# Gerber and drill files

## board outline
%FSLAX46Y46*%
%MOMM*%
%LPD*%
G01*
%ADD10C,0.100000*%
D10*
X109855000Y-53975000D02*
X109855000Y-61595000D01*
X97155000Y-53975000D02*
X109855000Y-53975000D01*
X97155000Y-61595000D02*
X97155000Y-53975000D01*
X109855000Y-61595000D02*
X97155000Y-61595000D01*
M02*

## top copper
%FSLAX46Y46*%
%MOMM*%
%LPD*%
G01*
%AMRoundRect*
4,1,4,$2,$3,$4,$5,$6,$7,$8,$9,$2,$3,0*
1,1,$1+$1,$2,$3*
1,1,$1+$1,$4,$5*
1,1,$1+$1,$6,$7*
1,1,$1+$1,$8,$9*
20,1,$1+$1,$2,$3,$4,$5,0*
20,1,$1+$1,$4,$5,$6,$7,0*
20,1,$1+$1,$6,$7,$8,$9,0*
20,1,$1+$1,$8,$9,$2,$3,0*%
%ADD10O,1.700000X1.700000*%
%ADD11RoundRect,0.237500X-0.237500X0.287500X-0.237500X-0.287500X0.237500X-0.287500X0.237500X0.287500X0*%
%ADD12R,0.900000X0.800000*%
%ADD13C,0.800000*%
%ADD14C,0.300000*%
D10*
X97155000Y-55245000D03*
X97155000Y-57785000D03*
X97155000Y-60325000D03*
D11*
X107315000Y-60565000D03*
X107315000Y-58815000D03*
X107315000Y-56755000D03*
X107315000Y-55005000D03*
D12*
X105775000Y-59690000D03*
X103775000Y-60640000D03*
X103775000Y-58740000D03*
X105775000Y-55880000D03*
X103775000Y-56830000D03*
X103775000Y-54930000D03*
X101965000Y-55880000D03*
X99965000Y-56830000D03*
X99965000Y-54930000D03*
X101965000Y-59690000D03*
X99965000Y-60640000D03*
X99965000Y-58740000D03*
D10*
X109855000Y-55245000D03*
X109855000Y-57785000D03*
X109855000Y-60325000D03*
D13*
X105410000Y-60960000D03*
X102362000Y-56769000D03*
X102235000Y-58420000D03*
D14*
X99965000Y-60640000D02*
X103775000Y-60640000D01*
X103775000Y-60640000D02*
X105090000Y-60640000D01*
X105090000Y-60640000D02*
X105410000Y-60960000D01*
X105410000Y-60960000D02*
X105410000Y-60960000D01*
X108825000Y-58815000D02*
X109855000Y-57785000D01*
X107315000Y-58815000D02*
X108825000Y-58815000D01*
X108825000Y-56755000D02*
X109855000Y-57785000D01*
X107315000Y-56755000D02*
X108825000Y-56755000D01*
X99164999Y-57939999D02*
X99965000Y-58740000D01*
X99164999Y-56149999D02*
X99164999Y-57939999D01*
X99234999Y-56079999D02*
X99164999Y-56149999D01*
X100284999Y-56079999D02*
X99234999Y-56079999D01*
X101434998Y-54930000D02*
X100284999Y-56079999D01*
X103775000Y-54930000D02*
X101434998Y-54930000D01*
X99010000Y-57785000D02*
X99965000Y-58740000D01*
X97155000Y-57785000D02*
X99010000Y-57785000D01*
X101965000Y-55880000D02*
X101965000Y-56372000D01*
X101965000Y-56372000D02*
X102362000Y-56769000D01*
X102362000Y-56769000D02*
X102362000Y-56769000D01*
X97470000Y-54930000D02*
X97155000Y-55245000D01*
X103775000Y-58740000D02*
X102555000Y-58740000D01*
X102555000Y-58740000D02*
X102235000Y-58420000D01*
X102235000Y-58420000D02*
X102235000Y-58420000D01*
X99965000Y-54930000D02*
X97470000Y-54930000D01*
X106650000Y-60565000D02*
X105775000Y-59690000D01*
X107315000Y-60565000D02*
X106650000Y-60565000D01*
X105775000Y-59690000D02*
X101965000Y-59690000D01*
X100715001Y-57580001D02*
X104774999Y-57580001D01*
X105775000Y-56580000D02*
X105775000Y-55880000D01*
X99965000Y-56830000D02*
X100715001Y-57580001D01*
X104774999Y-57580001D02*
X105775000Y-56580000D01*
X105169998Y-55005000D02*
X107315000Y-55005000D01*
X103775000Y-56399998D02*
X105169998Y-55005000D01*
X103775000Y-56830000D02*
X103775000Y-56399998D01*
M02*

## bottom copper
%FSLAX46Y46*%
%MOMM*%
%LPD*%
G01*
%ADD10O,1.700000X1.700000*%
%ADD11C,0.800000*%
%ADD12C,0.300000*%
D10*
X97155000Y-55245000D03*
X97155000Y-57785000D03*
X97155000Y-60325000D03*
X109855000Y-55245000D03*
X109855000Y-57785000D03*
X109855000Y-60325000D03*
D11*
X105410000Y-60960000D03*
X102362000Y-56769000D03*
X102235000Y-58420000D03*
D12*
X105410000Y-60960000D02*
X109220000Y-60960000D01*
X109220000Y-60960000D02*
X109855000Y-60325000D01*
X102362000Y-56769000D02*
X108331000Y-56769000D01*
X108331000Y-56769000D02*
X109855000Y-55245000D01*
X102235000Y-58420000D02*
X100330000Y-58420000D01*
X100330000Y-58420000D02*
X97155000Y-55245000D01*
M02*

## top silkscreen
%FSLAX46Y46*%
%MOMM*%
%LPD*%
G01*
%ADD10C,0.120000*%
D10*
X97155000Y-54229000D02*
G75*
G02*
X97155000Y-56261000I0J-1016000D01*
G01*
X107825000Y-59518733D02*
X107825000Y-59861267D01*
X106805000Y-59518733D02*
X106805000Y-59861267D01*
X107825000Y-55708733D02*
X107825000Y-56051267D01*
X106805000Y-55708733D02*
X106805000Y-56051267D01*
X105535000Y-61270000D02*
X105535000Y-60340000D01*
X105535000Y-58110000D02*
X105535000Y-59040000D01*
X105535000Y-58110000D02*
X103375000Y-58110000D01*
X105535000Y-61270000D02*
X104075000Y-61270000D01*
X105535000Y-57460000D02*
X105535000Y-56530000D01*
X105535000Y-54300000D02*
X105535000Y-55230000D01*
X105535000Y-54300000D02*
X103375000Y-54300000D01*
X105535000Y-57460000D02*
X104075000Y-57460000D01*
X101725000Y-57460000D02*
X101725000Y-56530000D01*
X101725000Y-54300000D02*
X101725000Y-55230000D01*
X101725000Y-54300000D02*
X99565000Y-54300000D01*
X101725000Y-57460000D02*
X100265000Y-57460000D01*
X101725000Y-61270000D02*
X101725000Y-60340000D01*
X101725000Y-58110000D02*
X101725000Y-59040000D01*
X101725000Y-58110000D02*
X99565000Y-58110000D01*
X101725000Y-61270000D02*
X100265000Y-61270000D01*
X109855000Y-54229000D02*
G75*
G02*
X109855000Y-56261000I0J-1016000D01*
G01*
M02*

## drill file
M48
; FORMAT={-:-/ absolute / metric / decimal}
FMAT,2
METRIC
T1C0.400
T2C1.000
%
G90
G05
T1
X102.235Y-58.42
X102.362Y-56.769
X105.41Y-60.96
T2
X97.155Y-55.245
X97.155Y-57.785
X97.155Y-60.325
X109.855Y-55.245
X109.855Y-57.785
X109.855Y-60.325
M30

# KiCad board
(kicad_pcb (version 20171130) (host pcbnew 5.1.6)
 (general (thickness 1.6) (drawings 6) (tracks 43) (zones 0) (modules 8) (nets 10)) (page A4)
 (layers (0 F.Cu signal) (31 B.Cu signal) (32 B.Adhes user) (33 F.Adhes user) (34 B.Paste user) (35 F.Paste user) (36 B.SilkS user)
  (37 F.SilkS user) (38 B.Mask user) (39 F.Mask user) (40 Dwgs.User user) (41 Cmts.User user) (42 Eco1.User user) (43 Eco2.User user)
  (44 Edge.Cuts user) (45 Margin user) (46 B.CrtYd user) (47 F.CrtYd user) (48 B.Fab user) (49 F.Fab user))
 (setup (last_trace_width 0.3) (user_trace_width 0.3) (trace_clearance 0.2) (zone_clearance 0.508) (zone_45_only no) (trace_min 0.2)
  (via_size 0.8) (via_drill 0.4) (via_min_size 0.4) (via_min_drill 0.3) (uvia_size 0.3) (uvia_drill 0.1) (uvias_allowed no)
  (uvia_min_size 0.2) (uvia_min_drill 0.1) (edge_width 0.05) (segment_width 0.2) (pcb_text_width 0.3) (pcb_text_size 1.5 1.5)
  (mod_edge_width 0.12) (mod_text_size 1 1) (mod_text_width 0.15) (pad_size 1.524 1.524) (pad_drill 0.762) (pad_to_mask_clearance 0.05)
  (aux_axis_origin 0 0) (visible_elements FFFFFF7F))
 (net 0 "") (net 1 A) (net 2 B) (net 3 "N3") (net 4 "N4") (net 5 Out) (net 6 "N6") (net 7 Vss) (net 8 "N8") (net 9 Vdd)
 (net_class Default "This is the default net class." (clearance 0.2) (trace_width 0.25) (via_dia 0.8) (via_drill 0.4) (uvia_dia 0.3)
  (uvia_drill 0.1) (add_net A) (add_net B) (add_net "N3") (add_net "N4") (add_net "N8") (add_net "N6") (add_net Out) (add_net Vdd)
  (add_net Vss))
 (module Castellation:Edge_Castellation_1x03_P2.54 (layer F.Cu) (at 97.155 55.245)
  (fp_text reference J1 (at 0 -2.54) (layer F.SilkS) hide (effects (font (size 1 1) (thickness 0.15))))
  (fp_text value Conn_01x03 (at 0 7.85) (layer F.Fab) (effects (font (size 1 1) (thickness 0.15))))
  (fp_arc (start 0 0) (end 0 1.016) (angle -180) (layer F.SilkS) (width 0.12))
  (pad 1 thru_hole oval (at 0 0) (size 1.7 1.7) (drill 1) (layers *.Cu *.Mask) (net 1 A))
  (pad 2 thru_hole oval (at 0 2.54) (size 1.7 1.7) (drill 1) (layers *.Cu *.Mask) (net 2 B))
  (pad 3 thru_hole oval (at 0 5.08) (size 1.7 1.7) (drill 1) (layers *.Cu *.Mask) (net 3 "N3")))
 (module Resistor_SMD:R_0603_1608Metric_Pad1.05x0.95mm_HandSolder (layer F.Cu) (at 107.315 59.69 270)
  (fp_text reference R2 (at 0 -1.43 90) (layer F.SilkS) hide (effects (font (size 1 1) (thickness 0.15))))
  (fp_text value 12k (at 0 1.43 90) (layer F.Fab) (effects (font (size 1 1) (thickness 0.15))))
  (fp_line (start -0.171267 -0.51) (end 0.171267 -0.51) (layer F.SilkS) (width 0.12))
  (fp_line (start -0.171267 0.51) (end 0.171267 0.51) (layer F.SilkS) (width 0.12))
  (pad 2 smd roundrect (at 0.875 0 270) (size 1.05 0.95) (layers F.Cu F.Paste F.Mask) (roundrect_rratio 0.25) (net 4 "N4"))
  (pad 1 smd roundrect (at -0.875 0 270) (size 1.05 0.95) (layers F.Cu F.Paste F.Mask) (roundrect_rratio 0.25) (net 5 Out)))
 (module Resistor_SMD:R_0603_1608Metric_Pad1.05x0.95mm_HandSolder (layer F.Cu) (at 107.315 55.88 270)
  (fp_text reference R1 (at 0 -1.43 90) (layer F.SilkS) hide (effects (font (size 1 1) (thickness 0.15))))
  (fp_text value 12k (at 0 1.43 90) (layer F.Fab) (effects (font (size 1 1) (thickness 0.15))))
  (fp_line (start -0.171267 -0.51) (end 0.171267 -0.51) (layer F.SilkS) (width 0.12))
  (fp_line (start -0.171267 0.51) (end 0.171267 0.51) (layer F.SilkS) (width 0.12))
  (pad 2 smd roundrect (at 0.875 0 270) (size 1.05 0.95) (layers F.Cu F.Paste F.Mask) (roundrect_rratio 0.25) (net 5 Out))
  (pad 1 smd roundrect (at -0.875 0 270) (size 1.05 0.95) (layers F.Cu F.Paste F.Mask) (roundrect_rratio 0.25) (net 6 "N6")))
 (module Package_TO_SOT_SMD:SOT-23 (layer F.Cu) (at 104.775 59.69)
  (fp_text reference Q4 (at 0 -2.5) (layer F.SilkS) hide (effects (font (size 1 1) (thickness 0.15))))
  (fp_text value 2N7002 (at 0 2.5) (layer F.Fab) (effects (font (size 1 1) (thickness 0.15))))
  (fp_line (start 0.76 1.58) (end 0.76 0.65) (layer F.SilkS) (width 0.12))
  (fp_line (start 0.76 -1.58) (end 0.76 -0.65) (layer F.SilkS) (width 0.12))
  (fp_line (start 0.76 -1.58) (end -1.4 -1.58) (layer F.SilkS) (width 0.12))
  (fp_line (start 0.76 1.58) (end -0.7 1.58) (layer F.SilkS) (width 0.12))
  (pad 3 smd rect (at 1 0) (size 0.9 0.8) (layers F.Cu F.Paste F.Mask) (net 4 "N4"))
  (pad 2 smd rect (at -1 0.95) (size 0.9 0.8) (layers F.Cu F.Paste F.Mask) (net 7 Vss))
  (pad 1 smd rect (at -1 -0.95) (size 0.9 0.8) (layers F.Cu F.Paste F.Mask) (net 1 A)))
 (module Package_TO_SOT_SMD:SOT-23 (layer F.Cu) (at 104.775 55.88)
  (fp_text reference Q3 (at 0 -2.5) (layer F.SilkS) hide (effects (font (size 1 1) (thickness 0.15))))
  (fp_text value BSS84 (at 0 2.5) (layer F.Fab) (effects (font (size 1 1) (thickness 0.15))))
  (fp_line (start 0.76 1.58) (end 0.76 0.65) (layer F.SilkS) (width 0.12))
  (fp_line (start 0.76 -1.58) (end 0.76 -0.65) (layer F.SilkS) (width 0.12))
  (fp_line (start 0.76 -1.58) (end -1.4 -1.58) (layer F.SilkS) (width 0.12))
  (fp_line (start 0.76 1.58) (end -0.7 1.58) (layer F.SilkS) (width 0.12))
  (pad 3 smd rect (at 1 0) (size 0.9 0.8) (layers F.Cu F.Paste F.Mask) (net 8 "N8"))
  (pad 2 smd rect (at -1 0.95) (size 0.9 0.8) (layers F.Cu F.Paste F.Mask) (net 6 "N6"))
  (pad 1 smd rect (at -1 -0.95) (size 0.9 0.8) (layers F.Cu F.Paste F.Mask) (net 2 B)))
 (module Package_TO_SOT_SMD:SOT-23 (layer F.Cu) (at 100.965 55.88)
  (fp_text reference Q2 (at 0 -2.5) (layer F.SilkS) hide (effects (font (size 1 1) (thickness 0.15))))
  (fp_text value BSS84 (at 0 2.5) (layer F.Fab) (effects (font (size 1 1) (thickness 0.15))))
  (fp_line (start 0.76 1.58) (end 0.76 0.65) (layer F.SilkS) (width 0.12))
  (fp_line (start 0.76 -1.58) (end 0.76 -0.65) (layer F.SilkS) (width 0.12))
  (fp_line (start 0.76 -1.58) (end -1.4 -1.58) (layer F.SilkS) (width 0.12))
  (fp_line (start 0.76 1.58) (end -0.7 1.58) (layer F.SilkS) (width 0.12))
  (pad 3 smd rect (at 1 0) (size 0.9 0.8) (layers F.Cu F.Paste F.Mask) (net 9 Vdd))
  (pad 2 smd rect (at -1 0.95) (size 0.9 0.8) (layers F.Cu F.Paste F.Mask) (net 8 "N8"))
  (pad 1 smd rect (at -1 -0.95) (size 0.9 0.8) (layers F.Cu F.Paste F.Mask) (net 1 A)))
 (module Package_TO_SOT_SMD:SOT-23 (layer F.Cu) (at 100.965 59.69)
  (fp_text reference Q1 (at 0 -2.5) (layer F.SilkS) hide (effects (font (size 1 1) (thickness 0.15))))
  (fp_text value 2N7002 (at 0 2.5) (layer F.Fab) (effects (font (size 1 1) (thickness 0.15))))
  (fp_line (start 0.76 1.58) (end 0.76 0.65) (layer F.SilkS) (width 0.12))
  (fp_line (start 0.76 -1.58) (end 0.76 -0.65) (layer F.SilkS) (width 0.12))
  (fp_line (start 0.76 -1.58) (end -1.4 -1.58) (layer F.SilkS) (width 0.12))
  (fp_line (start 0.76 1.58) (end -0.7 1.58) (layer F.SilkS) (width 0.12))
  (pad 3 smd rect (at 1 0) (size 0.9 0.8) (layers F.Cu F.Paste F.Mask) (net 4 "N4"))
  (pad 2 smd rect (at -1 0.95) (size 0.9 0.8) (layers F.Cu F.Paste F.Mask) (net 7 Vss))
  (pad 1 smd rect (at -1 -0.95) (size 0.9 0.8) (layers F.Cu F.Paste F.Mask) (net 2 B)))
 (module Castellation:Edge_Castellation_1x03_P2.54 (layer F.Cu) (at 109.855 55.245)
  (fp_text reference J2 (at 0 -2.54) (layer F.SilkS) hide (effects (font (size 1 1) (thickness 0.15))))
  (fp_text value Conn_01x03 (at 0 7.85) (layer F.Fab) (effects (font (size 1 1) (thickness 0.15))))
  (fp_arc (start 0 0) (end 0 1.016) (angle -180) (layer F.SilkS) (width 0.12))
  (pad 1 thru_hole oval (at 0 0) (size 1.7 1.7) (drill 1) (layers *.Cu *.Mask) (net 9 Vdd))
  (pad 2 thru_hole oval (at 0 2.54) (size 1.7 1.7) (drill 1) (layers *.Cu *.Mask) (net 5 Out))
  (pad 3 thru_hole oval (at 0 5.08) (size 1.7 1.7) (drill 1) (layers *.Cu *.Mask) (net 7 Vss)))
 (gr_line (start 109.855 53.975) (end 109.855 61.595) (layer Edge.Cuts) (width 0.1))
 (gr_line (start 97.155 53.975) (end 109.855 53.975) (layer Edge.Cuts) (width 0.1))
 (gr_line (start 97.155 61.595) (end 97.155 53.975) (layer Edge.Cuts) (width 0.1))
 (gr_line (start 109.855 61.595) (end 97.155 61.595) (layer Edge.Cuts) (width 0.1))
 (segment (start 99.965 60.64) (end 103.775 60.64) (width 0.3) (layer F.Cu) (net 7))
 (segment (start 103.775 60.64) (end 105.09 60.64) (width 0.3) (layer F.Cu) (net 7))
 (segment (start 105.09 60.64) (end 105.41 60.96) (width 0.3) (layer F.Cu) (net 7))
 (segment (start 105.41 60.96) (end 105.41 60.96) (width 0.3) (layer F.Cu) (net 7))
 (via (at 105.41 60.96) (size 0.8) (drill 0.4) (layers F.Cu B.Cu) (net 7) (status 1000000))
 (segment (start 105.41 60.96) (end 109.22 60.96) (width 0.3) (layer B.Cu) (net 7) (status 1000000))
 (segment (start 109.22 60.96) (end 109.855 60.325) (width 0.3) (layer B.Cu) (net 7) (status 1000000))
 (segment (start 108.825 58.815) (end 109.855 57.785) (width 0.3) (layer F.Cu) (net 5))
 (segment (start 107.315 58.815) (end 108.825 58.815) (width 0.3) (layer F.Cu) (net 5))
 (segment (start 108.825 56.755) (end 109.855 57.785) (width 0.3) (layer F.Cu) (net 5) (status 1000000))
 (segment (start 107.315 56.755) (end 108.825 56.755) (width 0.3) (layer F.Cu) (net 5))
 (segment (start 99.164999 57.939999) (end 99.965 58.74) (width 0.3) (layer F.Cu) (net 2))
 (segment (start 99.164999 56.149999) (end 99.164999 57.939999) (width 0.3) (layer F.Cu) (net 2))
 (segment (start 99.234999 56.079999) (end 99.164999 56.149999) (width 0.3) (layer F.Cu) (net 2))
 (segment (start 100.284999 56.079999) (end 99.234999 56.079999) (width 0.3) (layer F.Cu) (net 2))
 (segment (start 101.434998 54.93) (end 100.284999 56.079999) (width 0.3) (layer F.Cu) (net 2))
 (segment (start 103.775 54.93) (end 101.434998 54.93) (width 0.3) (layer F.Cu) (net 2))
 (segment (start 99.01 57.785) (end 99.965 58.74) (width 0.3) (layer F.Cu) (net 2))
 (segment (start 97.155 57.785) (end 99.01 57.785) (width 0.3) (layer F.Cu) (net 2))
 (segment (start 101.965 55.88) (end 101.965 56.372) (width 0.3) (layer F.Cu) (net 9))
 (segment (start 101.965 56.372) (end 102.362 56.769) (width 0.3) (layer F.Cu) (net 9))
 (segment (start 102.362 56.769) (end 102.362 56.769) (width 0.3) (layer F.Cu) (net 9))
 (via (at 102.362 56.769) (size 0.8) (drill 0.4) (layers F.Cu B.Cu) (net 9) (status 1000000))
 (segment (start 102.362 56.769) (end 108.331 56.769) (width 0.3) (layer B.Cu) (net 9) (status 1000000))
 (segment (start 108.331 56.769) (end 109.855 55.245) (width 0.3) (layer B.Cu) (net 9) (status 1000000))
 (segment (start 97.47 54.93) (end 97.155 55.245) (width 0.3) (layer F.Cu) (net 1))
 (segment (start 103.775 58.74) (end 102.555 58.74) (width 0.3) (layer F.Cu) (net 1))
 (segment (start 102.555 58.74) (end 102.235 58.42) (width 0.3) (layer F.Cu) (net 1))
 (segment (start 102.235 58.42) (end 102.235 58.42) (width 0.3) (layer F.Cu) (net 1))
 (segment (start 99.965 54.93) (end 97.47 54.93) (width 0.3) (layer F.Cu) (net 1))
 (segment (start 102.235 58.42) (end 100.33 58.42) (width 0.3) (layer B.Cu) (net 1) (status 1000000))
 (via (at 102.235 58.42) (size 0.8) (drill 0.4) (layers F.Cu B.Cu) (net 1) (status 1000000))
 (segment (start 100.33 58.42) (end 97.155 55.245) (width 0.3) (layer B.Cu) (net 1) (status 1000000))
 (segment (start 106.65 60.565) (end 105.775 59.69) (width 0.3) (layer F.Cu) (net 4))
 (segment (start 107.315 60.565) (end 106.65 60.565) (width 0.3) (layer F.Cu) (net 4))
 (segment (start 105.775 59.69) (end 101.965 59.69) (width 0.3) (layer F.Cu) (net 4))
 (segment (start 100.715001 57.580001) (end 104.774999 57.580001) (width 0.3) (layer F.Cu) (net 8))
 (segment (start 105.775 56.58) (end 105.775 55.88) (width 0.3) (layer F.Cu) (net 8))
 (segment (start 99.965 56.83) (end 100.715001 57.580001) (width 0.3) (layer F.Cu) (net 8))
 (segment (start 104.774999 57.580001) (end 105.775 56.58) (width 0.3) (layer F.Cu) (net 8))
 (segment (start 105.169998 55.005) (end 107.315 55.005) (width 0.3) (layer F.Cu) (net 6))
 (segment (start 103.775 56.399998) (end 105.169998 55.005) (width 0.3) (layer F.Cu) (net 6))
 (segment (start 103.775 56.83) (end 103.775 56.399998) (width 0.3) (layer F.Cu) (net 6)))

